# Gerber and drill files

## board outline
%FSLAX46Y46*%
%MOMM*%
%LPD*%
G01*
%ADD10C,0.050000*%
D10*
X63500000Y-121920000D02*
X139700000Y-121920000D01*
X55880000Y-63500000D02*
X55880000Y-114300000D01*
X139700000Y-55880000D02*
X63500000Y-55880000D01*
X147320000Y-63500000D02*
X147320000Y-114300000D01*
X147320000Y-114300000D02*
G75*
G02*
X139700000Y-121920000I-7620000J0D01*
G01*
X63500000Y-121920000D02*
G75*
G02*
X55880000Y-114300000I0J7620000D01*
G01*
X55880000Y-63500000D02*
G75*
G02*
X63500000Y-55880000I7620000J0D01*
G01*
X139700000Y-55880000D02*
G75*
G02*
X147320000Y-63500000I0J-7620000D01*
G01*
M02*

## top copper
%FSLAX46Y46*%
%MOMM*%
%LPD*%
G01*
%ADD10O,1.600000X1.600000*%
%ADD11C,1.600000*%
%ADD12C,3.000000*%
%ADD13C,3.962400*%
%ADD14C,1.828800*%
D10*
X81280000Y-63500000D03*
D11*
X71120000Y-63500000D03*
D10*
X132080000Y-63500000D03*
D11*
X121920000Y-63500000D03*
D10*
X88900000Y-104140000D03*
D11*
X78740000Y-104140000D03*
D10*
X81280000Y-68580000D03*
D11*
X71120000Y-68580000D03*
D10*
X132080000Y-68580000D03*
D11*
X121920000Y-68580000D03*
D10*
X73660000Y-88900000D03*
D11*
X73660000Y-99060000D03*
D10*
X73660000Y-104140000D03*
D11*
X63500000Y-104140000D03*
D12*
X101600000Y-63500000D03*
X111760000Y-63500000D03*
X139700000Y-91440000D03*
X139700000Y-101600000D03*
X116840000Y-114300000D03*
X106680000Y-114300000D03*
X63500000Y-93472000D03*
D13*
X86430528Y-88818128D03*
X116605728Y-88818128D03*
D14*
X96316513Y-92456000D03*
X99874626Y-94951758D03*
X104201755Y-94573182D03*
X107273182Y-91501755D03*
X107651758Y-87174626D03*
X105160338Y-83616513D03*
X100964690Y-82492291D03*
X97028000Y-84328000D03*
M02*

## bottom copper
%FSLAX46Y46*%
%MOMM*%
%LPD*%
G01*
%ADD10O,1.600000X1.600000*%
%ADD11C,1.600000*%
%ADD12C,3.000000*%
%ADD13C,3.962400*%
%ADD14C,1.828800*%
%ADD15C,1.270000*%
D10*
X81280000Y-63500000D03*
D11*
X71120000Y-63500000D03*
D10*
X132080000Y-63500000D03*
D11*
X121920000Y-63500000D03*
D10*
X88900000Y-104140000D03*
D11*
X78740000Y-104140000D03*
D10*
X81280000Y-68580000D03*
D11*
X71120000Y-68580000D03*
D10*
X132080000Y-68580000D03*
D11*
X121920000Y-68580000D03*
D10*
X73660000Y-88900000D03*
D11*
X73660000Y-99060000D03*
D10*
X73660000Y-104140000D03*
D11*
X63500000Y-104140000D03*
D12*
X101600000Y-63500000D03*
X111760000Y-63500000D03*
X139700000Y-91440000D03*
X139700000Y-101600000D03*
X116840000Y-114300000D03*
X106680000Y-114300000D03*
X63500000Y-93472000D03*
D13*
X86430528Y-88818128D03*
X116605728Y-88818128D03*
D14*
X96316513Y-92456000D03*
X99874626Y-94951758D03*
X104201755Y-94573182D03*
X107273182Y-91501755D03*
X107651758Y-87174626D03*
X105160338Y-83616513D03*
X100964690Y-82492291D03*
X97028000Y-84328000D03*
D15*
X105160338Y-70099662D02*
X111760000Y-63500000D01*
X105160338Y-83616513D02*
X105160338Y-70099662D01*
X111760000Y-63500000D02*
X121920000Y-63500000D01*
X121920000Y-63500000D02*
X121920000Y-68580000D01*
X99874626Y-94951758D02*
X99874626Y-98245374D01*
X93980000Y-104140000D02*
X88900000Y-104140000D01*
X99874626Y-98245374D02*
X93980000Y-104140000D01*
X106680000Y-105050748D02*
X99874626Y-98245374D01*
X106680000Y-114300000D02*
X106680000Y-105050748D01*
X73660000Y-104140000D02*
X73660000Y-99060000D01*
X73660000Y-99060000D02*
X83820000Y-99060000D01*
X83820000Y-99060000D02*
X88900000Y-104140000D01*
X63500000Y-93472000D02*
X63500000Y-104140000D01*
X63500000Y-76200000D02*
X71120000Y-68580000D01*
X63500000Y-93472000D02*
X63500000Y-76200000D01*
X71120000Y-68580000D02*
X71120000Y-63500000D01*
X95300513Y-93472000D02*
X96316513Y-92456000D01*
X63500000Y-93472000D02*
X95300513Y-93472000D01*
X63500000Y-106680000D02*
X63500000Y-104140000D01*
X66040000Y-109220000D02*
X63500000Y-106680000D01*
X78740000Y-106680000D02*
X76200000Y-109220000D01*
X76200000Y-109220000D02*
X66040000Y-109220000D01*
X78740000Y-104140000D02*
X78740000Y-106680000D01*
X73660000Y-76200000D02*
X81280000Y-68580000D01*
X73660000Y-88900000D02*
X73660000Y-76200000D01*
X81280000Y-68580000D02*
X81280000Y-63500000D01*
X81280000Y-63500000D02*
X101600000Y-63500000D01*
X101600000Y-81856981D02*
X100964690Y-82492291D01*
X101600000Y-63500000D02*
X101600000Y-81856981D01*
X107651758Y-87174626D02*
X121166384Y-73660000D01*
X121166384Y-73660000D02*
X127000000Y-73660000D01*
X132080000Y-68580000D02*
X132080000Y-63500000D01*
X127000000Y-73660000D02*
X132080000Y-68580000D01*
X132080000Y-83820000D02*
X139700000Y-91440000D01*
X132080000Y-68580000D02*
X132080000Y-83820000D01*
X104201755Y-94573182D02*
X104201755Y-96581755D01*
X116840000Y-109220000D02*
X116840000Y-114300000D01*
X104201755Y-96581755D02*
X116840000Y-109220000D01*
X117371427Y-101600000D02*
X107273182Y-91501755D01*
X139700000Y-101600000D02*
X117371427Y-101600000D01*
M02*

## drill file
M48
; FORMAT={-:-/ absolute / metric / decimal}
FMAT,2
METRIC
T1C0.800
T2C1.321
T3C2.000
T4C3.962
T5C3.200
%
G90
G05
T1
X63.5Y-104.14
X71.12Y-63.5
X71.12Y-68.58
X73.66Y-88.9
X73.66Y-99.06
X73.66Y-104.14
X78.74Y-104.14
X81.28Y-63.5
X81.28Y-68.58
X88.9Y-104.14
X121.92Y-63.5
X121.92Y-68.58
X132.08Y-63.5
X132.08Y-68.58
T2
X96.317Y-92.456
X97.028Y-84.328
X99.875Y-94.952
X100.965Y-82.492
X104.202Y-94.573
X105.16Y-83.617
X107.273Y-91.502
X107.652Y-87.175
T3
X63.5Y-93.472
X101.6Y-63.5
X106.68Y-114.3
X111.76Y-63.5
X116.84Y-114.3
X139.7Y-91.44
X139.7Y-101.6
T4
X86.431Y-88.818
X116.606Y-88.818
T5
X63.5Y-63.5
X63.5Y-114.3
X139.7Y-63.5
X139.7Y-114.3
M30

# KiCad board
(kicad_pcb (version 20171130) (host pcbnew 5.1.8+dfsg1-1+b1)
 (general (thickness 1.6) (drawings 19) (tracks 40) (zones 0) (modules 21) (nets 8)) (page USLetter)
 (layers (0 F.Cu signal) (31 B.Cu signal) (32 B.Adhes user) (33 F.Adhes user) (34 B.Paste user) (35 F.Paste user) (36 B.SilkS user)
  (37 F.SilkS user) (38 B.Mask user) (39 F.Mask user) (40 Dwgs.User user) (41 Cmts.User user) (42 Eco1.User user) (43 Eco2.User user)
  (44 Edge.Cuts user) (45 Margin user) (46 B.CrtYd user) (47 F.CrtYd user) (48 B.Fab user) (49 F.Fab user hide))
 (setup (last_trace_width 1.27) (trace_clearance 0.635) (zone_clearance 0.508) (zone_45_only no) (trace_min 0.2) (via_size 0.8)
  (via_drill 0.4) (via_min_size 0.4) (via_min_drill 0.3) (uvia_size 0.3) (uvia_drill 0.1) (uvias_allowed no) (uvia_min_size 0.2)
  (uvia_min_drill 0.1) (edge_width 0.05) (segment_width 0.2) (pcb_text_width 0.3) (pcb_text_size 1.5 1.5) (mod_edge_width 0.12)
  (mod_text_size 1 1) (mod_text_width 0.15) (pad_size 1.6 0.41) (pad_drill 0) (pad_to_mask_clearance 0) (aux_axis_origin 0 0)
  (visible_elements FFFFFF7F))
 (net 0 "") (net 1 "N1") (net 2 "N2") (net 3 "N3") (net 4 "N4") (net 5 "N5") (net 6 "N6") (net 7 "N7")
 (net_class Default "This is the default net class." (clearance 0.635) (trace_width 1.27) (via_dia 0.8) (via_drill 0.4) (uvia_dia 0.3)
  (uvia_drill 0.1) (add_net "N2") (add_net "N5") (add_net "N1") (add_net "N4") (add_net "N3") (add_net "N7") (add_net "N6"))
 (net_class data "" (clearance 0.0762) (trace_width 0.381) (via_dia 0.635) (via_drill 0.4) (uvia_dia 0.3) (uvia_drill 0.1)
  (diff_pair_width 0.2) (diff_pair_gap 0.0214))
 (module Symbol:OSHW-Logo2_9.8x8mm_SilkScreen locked (layer B.Cu) (at 81.28 110.49 180)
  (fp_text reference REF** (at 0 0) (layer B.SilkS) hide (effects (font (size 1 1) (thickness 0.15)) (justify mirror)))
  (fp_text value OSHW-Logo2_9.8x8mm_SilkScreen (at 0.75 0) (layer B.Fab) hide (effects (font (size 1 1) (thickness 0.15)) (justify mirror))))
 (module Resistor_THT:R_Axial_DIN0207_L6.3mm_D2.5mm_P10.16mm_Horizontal (layer F.Cu) (at 71.12 63.5)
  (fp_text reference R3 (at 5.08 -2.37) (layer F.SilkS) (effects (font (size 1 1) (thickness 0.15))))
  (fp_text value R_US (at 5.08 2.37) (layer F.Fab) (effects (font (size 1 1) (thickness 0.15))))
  (pad 2 thru_hole oval (at 10.16 0) (size 1.6 1.6) (drill 0.8) (layers *.Cu *.Mask) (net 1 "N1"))
  (pad 1 thru_hole circle (at 0 0) (size 1.6 1.6) (drill 0.8) (layers *.Cu *.Mask) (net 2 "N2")))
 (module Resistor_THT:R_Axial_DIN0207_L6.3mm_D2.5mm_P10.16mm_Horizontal (layer F.Cu) (at 121.92 63.5)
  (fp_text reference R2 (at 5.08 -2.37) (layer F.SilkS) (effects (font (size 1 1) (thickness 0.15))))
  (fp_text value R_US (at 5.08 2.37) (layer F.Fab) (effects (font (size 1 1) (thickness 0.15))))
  (pad 2 thru_hole oval (at 10.16 0) (size 1.6 1.6) (drill 0.8) (layers *.Cu *.Mask) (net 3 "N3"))
  (pad 1 thru_hole circle (at 0 0) (size 1.6 1.6) (drill 0.8) (layers *.Cu *.Mask) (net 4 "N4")))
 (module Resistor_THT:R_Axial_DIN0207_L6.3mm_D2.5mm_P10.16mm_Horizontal (layer F.Cu) (at 78.74 104.14)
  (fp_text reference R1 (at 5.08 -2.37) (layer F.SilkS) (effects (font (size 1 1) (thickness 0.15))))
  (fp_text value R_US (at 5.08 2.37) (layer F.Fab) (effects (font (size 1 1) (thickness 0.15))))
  (pad 2 thru_hole oval (at 10.16 0) (size 1.6 1.6) (drill 0.8) (layers *.Cu *.Mask) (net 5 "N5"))
  (pad 1 thru_hole circle (at 0 0) (size 1.6 1.6) (drill 0.8) (layers *.Cu *.Mask) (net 2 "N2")))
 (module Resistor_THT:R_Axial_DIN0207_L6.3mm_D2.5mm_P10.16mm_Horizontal (layer F.Cu) (at 71.12 68.58)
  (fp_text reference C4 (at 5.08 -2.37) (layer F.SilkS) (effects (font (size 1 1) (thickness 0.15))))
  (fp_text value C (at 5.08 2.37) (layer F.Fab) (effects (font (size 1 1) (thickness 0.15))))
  (pad 2 thru_hole oval (at 10.16 0) (size 1.6 1.6) (drill 0.8) (layers *.Cu *.Mask) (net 1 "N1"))
  (pad 1 thru_hole circle (at 0 0) (size 1.6 1.6) (drill 0.8) (layers *.Cu *.Mask) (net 2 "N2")))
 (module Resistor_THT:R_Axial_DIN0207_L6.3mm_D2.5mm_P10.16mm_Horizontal (layer F.Cu) (at 121.92 68.58)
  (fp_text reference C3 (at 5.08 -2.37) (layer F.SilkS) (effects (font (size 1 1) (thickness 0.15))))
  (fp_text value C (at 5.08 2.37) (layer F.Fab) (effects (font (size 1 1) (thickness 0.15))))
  (pad 2 thru_hole oval (at 10.16 0) (size 1.6 1.6) (drill 0.8) (layers *.Cu *.Mask) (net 3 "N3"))
  (pad 1 thru_hole circle (at 0 0) (size 1.6 1.6) (drill 0.8) (layers *.Cu *.Mask) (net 4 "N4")))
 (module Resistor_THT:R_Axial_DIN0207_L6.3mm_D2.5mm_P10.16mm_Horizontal (layer F.Cu) (at 73.66 99.06 90)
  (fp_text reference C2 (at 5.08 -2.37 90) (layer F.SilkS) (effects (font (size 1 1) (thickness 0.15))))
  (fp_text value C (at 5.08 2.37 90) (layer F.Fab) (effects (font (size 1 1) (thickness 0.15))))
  (pad 2 thru_hole oval (at 10.16 0 90) (size 1.6 1.6) (drill 0.8) (layers *.Cu *.Mask) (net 1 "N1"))
  (pad 1 thru_hole circle (at 0 0 90) (size 1.6 1.6) (drill 0.8) (layers *.Cu *.Mask) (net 5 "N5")))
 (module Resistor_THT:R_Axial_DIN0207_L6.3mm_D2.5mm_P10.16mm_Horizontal (layer F.Cu) (at 63.5 104.14)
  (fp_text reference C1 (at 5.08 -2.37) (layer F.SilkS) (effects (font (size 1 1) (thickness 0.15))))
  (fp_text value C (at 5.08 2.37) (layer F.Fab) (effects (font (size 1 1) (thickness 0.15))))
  (pad 2 thru_hole oval (at 10.16 0) (size 1.6 1.6) (drill 0.8) (layers *.Cu *.Mask) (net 5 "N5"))
  (pad 1 thru_hole circle (at 0 0) (size 1.6 1.6) (drill 0.8) (layers *.Cu *.Mask) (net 2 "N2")))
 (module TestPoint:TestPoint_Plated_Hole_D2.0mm (layer F.Cu) (at 101.6 63.5 180)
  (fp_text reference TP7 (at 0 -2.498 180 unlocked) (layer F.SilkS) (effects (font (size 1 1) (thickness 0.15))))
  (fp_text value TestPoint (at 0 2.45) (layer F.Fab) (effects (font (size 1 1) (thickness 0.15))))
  (pad 1 thru_hole circle (at 0 0 180) (size 3 3) (drill 2) (layers *.Cu *.Mask) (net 1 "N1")))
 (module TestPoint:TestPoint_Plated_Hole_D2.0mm (layer F.Cu) (at 111.76 63.5 180)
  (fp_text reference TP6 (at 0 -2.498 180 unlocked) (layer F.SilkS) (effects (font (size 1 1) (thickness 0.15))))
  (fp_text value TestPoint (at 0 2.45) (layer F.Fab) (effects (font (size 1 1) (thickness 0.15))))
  (pad 1 thru_hole circle (at 0 0 180) (size 3 3) (drill 2) (layers *.Cu *.Mask) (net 4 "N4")))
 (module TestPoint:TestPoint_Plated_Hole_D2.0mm (layer F.Cu) (at 139.7 91.44 90)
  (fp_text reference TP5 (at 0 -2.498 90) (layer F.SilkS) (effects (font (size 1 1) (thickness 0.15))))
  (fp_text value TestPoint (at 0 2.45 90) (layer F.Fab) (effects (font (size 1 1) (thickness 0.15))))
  (pad 1 thru_hole circle (at 0 0 90) (size 3 3) (drill 2) (layers *.Cu *.Mask) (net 3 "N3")))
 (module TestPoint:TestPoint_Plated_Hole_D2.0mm (layer F.Cu) (at 139.7 101.6 90)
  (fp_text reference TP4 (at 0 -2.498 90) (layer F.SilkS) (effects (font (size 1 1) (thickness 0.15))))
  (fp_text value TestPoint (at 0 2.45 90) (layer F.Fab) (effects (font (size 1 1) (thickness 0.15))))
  (pad 1 thru_hole circle (at 0 0 90) (size 3 3) (drill 2) (layers *.Cu *.Mask) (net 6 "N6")))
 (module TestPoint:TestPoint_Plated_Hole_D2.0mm (layer F.Cu) (at 116.84 114.3)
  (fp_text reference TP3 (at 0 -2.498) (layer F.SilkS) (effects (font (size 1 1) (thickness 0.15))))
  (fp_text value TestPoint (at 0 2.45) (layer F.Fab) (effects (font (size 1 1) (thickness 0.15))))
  (pad 1 thru_hole circle (at 0 0) (size 3 3) (drill 2) (layers *.Cu *.Mask) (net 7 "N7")))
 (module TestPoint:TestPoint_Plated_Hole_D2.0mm (layer F.Cu) (at 106.68 114.3)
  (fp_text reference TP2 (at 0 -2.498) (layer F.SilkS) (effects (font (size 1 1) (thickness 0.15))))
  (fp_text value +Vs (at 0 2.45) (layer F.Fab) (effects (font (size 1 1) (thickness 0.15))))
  (pad 1 thru_hole circle (at 0 0) (size 3 3) (drill 2) (layers *.Cu *.Mask) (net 5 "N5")))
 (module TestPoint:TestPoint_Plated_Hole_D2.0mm (layer F.Cu) (at 63.5 93.472 270)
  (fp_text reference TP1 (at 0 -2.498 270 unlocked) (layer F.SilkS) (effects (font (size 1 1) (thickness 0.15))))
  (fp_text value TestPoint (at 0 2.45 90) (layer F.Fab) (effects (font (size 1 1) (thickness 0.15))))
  (pad 1 thru_hole circle (at 0 0 270) (size 3 3) (drill 2) (layers *.Cu *.Mask) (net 2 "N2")))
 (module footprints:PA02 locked (layer F.Cu) (at 97.028 84.328)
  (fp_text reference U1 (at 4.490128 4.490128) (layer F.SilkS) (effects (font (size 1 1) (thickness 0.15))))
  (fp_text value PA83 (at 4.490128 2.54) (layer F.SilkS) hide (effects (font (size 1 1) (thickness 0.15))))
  (pad 10 thru_hole circle (at -10.597472 4.490128) (size 3.9624 3.9624) (drill 3.9624) (layers *.Cu *.Mask))
  (pad 9 thru_hole circle (at 19.577728 4.490128) (size 3.9624 3.9624) (drill 3.9624) (layers *.Cu *.Mask))
  (pad 1 thru_hole circle (at -0.711487 8.128 80) (size 1.8288 1.8288) (drill 1.3208) (layers *.Cu *.Mask) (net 2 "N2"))
  (pad 2 thru_hole circle (at 2.846626 10.623758 120) (size 1.8288 1.8288) (drill 1.3208) (layers *.Cu *.Mask) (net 5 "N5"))
  (pad 3 thru_hole circle (at 7.173755 10.245182 160) (size 1.8288 1.8288) (drill 1.3208) (layers *.Cu *.Mask) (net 7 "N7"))
  (pad 4 thru_hole circle (at 10.245182 7.173755 200) (size 1.8288 1.8288) (drill 1.3208) (layers *.Cu *.Mask) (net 6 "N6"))
  (pad 5 thru_hole circle (at 10.623758 2.846626 240) (size 1.8288 1.8288) (drill 1.3208) (layers *.Cu *.Mask) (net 3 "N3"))
  (pad 6 thru_hole circle (at 8.132338 -0.711487 280) (size 1.8288 1.8288) (drill 1.3208) (layers *.Cu *.Mask) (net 4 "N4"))
  (pad 7 thru_hole circle (at 3.93669 -1.835709 320) (size 1.8288 1.8288) (drill 1.3208) (layers *.Cu *.Mask) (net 1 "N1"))
  (pad 8 thru_hole circle (at 0 0) (size 1.8288 1.8288) (drill 1.3208) (layers *.Cu *.Mask)))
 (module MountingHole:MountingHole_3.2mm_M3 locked (layer F.Cu) (at 63.5 114.3)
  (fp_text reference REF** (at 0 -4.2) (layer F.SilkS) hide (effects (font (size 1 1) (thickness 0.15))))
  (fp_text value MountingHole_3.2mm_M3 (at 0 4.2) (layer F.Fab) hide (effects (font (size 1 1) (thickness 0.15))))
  (pad 1 np_thru_hole circle (at 0 0) (size 3.2 3.2) (drill 3.2) (layers *.Cu *.Mask)))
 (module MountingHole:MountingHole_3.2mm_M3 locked (layer F.Cu) (at 139.7 114.3)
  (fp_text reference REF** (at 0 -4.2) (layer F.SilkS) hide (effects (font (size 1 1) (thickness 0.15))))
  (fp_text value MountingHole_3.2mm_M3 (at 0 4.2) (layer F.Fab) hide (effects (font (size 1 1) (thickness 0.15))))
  (pad 1 np_thru_hole circle (at 0 0) (size 3.2 3.2) (drill 3.2) (layers *.Cu *.Mask)))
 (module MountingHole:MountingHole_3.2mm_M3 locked (layer F.Cu) (at 63.5 63.5)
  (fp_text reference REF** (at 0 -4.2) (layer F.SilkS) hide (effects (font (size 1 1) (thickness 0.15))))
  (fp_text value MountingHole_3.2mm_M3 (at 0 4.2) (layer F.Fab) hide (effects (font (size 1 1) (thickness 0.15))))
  (pad 1 np_thru_hole circle (at 0 0) (size 3.2 3.2) (drill 3.2) (layers *.Cu *.Mask)))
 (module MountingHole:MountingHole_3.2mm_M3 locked (layer F.Cu) (at 139.7 63.5)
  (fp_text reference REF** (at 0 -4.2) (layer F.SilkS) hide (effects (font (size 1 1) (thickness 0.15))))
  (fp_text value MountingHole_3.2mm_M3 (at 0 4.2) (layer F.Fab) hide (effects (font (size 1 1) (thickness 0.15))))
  (pad 1 np_thru_hole circle (at 0 0) (size 3.2 3.2) (drill 3.2) (layers *.Cu *.Mask)))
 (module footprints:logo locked (layer F.Cu) (at 73.66 114.3)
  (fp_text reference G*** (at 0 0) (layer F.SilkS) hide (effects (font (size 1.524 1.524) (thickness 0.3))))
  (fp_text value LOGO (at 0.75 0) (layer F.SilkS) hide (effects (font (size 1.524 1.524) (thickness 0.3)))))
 (gr_line (start 63.5 121.92) (end 139.7 121.92) (layer Edge.Cuts) (width 0.05))
 (gr_line (start 55.88 63.5) (end 55.88 114.3) (layer Edge.Cuts) (width 0.05))
 (gr_line (start 139.7 55.88) (end 63.5 55.88) (layer Edge.Cuts) (width 0.05))
 (gr_line (start 147.32 63.5) (end 147.32 114.3) (layer Edge.Cuts) (width 0.05))
 (gr_arc (start 139.7 114.3) (end 139.7 121.92) (angle -90) (layer Edge.Cuts) (width 0.05))
 (gr_arc (start 63.5 114.3) (end 55.88 114.3) (angle -90) (layer Edge.Cuts) (width 0.05))
 (gr_arc (start 63.5 63.5) (end 63.5 55.88) (angle -90) (layer Edge.Cuts) (width 0.05))
 (gr_arc (start 139.7 63.5) (end 147.32 63.5) (angle -90) (layer Edge.Cuts) (width 0.05))
 (segment (start 105.160338 70.099662) (end 111.76 63.5) (width 1.27) (layer B.Cu) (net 4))
 (segment (start 105.160338 83.616513) (end 105.160338 70.099662) (width 1.27) (layer B.Cu) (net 4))
 (segment (start 111.76 63.5) (end 121.92 63.5) (width 1.27) (layer B.Cu) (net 4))
 (segment (start 121.92 63.5) (end 121.92 68.58) (width 1.27) (layer B.Cu) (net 4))
 (segment (start 99.874626 94.951758) (end 99.874626 98.245374) (width 1.27) (layer B.Cu) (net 5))
 (segment (start 93.98 104.14) (end 88.9 104.14) (width 1.27) (layer B.Cu) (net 5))
 (segment (start 99.874626 98.245374) (end 93.98 104.14) (width 1.27) (layer B.Cu) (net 5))
 (segment (start 106.68 105.050748) (end 99.874626 98.245374) (width 1.27) (layer B.Cu) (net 5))
 (segment (start 106.68 114.3) (end 106.68 105.050748) (width 1.27) (layer B.Cu) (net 5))
 (segment (start 73.66 104.14) (end 73.66 99.06) (width 1.27) (layer B.Cu) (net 5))
 (segment (start 73.66 99.06) (end 83.82 99.06) (width 1.27) (layer B.Cu) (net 5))
 (segment (start 83.82 99.06) (end 88.9 104.14) (width 1.27) (layer B.Cu) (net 5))
 (segment (start 63.5 93.472) (end 63.5 104.14) (width 1.27) (layer B.Cu) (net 2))
 (segment (start 63.5 76.2) (end 71.12 68.58) (width 1.27) (layer B.Cu) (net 2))
 (segment (start 63.5 93.472) (end 63.5 76.2) (width 1.27) (layer B.Cu) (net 2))
 (segment (start 71.12 68.58) (end 71.12 63.5) (width 1.27) (layer B.Cu) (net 2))
 (segment (start 95.300513 93.472) (end 96.316513 92.456) (width 1.27) (layer B.Cu) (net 2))
 (segment (start 63.5 93.472) (end 95.300513 93.472) (width 1.27) (layer B.Cu) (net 2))
 (segment (start 63.5 106.68) (end 63.5 104.14) (width 1.27) (layer B.Cu) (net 2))
 (segment (start 66.04 109.22) (end 63.5 106.68) (width 1.27) (layer B.Cu) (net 2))
 (segment (start 78.74 106.68) (end 76.2 109.22) (width 1.27) (layer B.Cu) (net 2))
 (segment (start 76.2 109.22) (end 66.04 109.22) (width 1.27) (layer B.Cu) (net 2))
 (segment (start 78.74 104.14) (end 78.74 106.68) (width 1.27) (layer B.Cu) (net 2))
 (segment (start 73.66 76.2) (end 81.28 68.58) (width 1.27) (layer B.Cu) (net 1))
 (segment (start 73.66 88.9) (end 73.66 76.2) (width 1.27) (layer B.Cu) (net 1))
 (segment (start 81.28 68.58) (end 81.28 63.5) (width 1.27) (layer B.Cu) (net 1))
 (segment (start 81.28 63.5) (end 101.6 63.5) (width 1.27) (layer B.Cu) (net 1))
 (segment (start 101.6 81.856981) (end 100.96469 82.492291) (width 1.27) (layer B.Cu) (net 1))
 (segment (start 101.6 63.5) (end 101.6 81.856981) (width 1.27) (layer B.Cu) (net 1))
 (segment (start 107.651758 87.174626) (end 121.166384 73.66) (width 1.27) (layer B.Cu) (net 3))
 (segment (start 121.166384 73.66) (end 127 73.66) (width 1.27) (layer B.Cu) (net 3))
 (segment (start 132.08 68.58) (end 132.08 63.5) (width 1.27) (layer B.Cu) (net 3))
 (segment (start 127 73.66) (end 132.08 68.58) (width 1.27) (layer B.Cu) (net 3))
 (segment (start 132.08 83.82) (end 139.7 91.44) (width 1.27) (layer B.Cu) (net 3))
 (segment (start 132.08 68.58) (end 132.08 83.82) (width 1.27) (layer B.Cu) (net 3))
 (segment (start 104.201755 94.573182) (end 104.201755 96.581755) (width 1.27) (layer B.Cu) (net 7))
 (segment (start 116.84 109.22) (end 116.84 114.3) (width 1.27) (layer B.Cu) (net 7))
 (segment (start 104.201755 96.581755) (end 116.84 109.22) (width 1.27) (layer B.Cu) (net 7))
 (segment (start 117.371427 101.6) (end 107.273182 91.501755) (width 1.27) (layer B.Cu) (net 6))
 (segment (start 139.7 101.6) (end 117.371427 101.6) (width 1.27) (layer B.Cu) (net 6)))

